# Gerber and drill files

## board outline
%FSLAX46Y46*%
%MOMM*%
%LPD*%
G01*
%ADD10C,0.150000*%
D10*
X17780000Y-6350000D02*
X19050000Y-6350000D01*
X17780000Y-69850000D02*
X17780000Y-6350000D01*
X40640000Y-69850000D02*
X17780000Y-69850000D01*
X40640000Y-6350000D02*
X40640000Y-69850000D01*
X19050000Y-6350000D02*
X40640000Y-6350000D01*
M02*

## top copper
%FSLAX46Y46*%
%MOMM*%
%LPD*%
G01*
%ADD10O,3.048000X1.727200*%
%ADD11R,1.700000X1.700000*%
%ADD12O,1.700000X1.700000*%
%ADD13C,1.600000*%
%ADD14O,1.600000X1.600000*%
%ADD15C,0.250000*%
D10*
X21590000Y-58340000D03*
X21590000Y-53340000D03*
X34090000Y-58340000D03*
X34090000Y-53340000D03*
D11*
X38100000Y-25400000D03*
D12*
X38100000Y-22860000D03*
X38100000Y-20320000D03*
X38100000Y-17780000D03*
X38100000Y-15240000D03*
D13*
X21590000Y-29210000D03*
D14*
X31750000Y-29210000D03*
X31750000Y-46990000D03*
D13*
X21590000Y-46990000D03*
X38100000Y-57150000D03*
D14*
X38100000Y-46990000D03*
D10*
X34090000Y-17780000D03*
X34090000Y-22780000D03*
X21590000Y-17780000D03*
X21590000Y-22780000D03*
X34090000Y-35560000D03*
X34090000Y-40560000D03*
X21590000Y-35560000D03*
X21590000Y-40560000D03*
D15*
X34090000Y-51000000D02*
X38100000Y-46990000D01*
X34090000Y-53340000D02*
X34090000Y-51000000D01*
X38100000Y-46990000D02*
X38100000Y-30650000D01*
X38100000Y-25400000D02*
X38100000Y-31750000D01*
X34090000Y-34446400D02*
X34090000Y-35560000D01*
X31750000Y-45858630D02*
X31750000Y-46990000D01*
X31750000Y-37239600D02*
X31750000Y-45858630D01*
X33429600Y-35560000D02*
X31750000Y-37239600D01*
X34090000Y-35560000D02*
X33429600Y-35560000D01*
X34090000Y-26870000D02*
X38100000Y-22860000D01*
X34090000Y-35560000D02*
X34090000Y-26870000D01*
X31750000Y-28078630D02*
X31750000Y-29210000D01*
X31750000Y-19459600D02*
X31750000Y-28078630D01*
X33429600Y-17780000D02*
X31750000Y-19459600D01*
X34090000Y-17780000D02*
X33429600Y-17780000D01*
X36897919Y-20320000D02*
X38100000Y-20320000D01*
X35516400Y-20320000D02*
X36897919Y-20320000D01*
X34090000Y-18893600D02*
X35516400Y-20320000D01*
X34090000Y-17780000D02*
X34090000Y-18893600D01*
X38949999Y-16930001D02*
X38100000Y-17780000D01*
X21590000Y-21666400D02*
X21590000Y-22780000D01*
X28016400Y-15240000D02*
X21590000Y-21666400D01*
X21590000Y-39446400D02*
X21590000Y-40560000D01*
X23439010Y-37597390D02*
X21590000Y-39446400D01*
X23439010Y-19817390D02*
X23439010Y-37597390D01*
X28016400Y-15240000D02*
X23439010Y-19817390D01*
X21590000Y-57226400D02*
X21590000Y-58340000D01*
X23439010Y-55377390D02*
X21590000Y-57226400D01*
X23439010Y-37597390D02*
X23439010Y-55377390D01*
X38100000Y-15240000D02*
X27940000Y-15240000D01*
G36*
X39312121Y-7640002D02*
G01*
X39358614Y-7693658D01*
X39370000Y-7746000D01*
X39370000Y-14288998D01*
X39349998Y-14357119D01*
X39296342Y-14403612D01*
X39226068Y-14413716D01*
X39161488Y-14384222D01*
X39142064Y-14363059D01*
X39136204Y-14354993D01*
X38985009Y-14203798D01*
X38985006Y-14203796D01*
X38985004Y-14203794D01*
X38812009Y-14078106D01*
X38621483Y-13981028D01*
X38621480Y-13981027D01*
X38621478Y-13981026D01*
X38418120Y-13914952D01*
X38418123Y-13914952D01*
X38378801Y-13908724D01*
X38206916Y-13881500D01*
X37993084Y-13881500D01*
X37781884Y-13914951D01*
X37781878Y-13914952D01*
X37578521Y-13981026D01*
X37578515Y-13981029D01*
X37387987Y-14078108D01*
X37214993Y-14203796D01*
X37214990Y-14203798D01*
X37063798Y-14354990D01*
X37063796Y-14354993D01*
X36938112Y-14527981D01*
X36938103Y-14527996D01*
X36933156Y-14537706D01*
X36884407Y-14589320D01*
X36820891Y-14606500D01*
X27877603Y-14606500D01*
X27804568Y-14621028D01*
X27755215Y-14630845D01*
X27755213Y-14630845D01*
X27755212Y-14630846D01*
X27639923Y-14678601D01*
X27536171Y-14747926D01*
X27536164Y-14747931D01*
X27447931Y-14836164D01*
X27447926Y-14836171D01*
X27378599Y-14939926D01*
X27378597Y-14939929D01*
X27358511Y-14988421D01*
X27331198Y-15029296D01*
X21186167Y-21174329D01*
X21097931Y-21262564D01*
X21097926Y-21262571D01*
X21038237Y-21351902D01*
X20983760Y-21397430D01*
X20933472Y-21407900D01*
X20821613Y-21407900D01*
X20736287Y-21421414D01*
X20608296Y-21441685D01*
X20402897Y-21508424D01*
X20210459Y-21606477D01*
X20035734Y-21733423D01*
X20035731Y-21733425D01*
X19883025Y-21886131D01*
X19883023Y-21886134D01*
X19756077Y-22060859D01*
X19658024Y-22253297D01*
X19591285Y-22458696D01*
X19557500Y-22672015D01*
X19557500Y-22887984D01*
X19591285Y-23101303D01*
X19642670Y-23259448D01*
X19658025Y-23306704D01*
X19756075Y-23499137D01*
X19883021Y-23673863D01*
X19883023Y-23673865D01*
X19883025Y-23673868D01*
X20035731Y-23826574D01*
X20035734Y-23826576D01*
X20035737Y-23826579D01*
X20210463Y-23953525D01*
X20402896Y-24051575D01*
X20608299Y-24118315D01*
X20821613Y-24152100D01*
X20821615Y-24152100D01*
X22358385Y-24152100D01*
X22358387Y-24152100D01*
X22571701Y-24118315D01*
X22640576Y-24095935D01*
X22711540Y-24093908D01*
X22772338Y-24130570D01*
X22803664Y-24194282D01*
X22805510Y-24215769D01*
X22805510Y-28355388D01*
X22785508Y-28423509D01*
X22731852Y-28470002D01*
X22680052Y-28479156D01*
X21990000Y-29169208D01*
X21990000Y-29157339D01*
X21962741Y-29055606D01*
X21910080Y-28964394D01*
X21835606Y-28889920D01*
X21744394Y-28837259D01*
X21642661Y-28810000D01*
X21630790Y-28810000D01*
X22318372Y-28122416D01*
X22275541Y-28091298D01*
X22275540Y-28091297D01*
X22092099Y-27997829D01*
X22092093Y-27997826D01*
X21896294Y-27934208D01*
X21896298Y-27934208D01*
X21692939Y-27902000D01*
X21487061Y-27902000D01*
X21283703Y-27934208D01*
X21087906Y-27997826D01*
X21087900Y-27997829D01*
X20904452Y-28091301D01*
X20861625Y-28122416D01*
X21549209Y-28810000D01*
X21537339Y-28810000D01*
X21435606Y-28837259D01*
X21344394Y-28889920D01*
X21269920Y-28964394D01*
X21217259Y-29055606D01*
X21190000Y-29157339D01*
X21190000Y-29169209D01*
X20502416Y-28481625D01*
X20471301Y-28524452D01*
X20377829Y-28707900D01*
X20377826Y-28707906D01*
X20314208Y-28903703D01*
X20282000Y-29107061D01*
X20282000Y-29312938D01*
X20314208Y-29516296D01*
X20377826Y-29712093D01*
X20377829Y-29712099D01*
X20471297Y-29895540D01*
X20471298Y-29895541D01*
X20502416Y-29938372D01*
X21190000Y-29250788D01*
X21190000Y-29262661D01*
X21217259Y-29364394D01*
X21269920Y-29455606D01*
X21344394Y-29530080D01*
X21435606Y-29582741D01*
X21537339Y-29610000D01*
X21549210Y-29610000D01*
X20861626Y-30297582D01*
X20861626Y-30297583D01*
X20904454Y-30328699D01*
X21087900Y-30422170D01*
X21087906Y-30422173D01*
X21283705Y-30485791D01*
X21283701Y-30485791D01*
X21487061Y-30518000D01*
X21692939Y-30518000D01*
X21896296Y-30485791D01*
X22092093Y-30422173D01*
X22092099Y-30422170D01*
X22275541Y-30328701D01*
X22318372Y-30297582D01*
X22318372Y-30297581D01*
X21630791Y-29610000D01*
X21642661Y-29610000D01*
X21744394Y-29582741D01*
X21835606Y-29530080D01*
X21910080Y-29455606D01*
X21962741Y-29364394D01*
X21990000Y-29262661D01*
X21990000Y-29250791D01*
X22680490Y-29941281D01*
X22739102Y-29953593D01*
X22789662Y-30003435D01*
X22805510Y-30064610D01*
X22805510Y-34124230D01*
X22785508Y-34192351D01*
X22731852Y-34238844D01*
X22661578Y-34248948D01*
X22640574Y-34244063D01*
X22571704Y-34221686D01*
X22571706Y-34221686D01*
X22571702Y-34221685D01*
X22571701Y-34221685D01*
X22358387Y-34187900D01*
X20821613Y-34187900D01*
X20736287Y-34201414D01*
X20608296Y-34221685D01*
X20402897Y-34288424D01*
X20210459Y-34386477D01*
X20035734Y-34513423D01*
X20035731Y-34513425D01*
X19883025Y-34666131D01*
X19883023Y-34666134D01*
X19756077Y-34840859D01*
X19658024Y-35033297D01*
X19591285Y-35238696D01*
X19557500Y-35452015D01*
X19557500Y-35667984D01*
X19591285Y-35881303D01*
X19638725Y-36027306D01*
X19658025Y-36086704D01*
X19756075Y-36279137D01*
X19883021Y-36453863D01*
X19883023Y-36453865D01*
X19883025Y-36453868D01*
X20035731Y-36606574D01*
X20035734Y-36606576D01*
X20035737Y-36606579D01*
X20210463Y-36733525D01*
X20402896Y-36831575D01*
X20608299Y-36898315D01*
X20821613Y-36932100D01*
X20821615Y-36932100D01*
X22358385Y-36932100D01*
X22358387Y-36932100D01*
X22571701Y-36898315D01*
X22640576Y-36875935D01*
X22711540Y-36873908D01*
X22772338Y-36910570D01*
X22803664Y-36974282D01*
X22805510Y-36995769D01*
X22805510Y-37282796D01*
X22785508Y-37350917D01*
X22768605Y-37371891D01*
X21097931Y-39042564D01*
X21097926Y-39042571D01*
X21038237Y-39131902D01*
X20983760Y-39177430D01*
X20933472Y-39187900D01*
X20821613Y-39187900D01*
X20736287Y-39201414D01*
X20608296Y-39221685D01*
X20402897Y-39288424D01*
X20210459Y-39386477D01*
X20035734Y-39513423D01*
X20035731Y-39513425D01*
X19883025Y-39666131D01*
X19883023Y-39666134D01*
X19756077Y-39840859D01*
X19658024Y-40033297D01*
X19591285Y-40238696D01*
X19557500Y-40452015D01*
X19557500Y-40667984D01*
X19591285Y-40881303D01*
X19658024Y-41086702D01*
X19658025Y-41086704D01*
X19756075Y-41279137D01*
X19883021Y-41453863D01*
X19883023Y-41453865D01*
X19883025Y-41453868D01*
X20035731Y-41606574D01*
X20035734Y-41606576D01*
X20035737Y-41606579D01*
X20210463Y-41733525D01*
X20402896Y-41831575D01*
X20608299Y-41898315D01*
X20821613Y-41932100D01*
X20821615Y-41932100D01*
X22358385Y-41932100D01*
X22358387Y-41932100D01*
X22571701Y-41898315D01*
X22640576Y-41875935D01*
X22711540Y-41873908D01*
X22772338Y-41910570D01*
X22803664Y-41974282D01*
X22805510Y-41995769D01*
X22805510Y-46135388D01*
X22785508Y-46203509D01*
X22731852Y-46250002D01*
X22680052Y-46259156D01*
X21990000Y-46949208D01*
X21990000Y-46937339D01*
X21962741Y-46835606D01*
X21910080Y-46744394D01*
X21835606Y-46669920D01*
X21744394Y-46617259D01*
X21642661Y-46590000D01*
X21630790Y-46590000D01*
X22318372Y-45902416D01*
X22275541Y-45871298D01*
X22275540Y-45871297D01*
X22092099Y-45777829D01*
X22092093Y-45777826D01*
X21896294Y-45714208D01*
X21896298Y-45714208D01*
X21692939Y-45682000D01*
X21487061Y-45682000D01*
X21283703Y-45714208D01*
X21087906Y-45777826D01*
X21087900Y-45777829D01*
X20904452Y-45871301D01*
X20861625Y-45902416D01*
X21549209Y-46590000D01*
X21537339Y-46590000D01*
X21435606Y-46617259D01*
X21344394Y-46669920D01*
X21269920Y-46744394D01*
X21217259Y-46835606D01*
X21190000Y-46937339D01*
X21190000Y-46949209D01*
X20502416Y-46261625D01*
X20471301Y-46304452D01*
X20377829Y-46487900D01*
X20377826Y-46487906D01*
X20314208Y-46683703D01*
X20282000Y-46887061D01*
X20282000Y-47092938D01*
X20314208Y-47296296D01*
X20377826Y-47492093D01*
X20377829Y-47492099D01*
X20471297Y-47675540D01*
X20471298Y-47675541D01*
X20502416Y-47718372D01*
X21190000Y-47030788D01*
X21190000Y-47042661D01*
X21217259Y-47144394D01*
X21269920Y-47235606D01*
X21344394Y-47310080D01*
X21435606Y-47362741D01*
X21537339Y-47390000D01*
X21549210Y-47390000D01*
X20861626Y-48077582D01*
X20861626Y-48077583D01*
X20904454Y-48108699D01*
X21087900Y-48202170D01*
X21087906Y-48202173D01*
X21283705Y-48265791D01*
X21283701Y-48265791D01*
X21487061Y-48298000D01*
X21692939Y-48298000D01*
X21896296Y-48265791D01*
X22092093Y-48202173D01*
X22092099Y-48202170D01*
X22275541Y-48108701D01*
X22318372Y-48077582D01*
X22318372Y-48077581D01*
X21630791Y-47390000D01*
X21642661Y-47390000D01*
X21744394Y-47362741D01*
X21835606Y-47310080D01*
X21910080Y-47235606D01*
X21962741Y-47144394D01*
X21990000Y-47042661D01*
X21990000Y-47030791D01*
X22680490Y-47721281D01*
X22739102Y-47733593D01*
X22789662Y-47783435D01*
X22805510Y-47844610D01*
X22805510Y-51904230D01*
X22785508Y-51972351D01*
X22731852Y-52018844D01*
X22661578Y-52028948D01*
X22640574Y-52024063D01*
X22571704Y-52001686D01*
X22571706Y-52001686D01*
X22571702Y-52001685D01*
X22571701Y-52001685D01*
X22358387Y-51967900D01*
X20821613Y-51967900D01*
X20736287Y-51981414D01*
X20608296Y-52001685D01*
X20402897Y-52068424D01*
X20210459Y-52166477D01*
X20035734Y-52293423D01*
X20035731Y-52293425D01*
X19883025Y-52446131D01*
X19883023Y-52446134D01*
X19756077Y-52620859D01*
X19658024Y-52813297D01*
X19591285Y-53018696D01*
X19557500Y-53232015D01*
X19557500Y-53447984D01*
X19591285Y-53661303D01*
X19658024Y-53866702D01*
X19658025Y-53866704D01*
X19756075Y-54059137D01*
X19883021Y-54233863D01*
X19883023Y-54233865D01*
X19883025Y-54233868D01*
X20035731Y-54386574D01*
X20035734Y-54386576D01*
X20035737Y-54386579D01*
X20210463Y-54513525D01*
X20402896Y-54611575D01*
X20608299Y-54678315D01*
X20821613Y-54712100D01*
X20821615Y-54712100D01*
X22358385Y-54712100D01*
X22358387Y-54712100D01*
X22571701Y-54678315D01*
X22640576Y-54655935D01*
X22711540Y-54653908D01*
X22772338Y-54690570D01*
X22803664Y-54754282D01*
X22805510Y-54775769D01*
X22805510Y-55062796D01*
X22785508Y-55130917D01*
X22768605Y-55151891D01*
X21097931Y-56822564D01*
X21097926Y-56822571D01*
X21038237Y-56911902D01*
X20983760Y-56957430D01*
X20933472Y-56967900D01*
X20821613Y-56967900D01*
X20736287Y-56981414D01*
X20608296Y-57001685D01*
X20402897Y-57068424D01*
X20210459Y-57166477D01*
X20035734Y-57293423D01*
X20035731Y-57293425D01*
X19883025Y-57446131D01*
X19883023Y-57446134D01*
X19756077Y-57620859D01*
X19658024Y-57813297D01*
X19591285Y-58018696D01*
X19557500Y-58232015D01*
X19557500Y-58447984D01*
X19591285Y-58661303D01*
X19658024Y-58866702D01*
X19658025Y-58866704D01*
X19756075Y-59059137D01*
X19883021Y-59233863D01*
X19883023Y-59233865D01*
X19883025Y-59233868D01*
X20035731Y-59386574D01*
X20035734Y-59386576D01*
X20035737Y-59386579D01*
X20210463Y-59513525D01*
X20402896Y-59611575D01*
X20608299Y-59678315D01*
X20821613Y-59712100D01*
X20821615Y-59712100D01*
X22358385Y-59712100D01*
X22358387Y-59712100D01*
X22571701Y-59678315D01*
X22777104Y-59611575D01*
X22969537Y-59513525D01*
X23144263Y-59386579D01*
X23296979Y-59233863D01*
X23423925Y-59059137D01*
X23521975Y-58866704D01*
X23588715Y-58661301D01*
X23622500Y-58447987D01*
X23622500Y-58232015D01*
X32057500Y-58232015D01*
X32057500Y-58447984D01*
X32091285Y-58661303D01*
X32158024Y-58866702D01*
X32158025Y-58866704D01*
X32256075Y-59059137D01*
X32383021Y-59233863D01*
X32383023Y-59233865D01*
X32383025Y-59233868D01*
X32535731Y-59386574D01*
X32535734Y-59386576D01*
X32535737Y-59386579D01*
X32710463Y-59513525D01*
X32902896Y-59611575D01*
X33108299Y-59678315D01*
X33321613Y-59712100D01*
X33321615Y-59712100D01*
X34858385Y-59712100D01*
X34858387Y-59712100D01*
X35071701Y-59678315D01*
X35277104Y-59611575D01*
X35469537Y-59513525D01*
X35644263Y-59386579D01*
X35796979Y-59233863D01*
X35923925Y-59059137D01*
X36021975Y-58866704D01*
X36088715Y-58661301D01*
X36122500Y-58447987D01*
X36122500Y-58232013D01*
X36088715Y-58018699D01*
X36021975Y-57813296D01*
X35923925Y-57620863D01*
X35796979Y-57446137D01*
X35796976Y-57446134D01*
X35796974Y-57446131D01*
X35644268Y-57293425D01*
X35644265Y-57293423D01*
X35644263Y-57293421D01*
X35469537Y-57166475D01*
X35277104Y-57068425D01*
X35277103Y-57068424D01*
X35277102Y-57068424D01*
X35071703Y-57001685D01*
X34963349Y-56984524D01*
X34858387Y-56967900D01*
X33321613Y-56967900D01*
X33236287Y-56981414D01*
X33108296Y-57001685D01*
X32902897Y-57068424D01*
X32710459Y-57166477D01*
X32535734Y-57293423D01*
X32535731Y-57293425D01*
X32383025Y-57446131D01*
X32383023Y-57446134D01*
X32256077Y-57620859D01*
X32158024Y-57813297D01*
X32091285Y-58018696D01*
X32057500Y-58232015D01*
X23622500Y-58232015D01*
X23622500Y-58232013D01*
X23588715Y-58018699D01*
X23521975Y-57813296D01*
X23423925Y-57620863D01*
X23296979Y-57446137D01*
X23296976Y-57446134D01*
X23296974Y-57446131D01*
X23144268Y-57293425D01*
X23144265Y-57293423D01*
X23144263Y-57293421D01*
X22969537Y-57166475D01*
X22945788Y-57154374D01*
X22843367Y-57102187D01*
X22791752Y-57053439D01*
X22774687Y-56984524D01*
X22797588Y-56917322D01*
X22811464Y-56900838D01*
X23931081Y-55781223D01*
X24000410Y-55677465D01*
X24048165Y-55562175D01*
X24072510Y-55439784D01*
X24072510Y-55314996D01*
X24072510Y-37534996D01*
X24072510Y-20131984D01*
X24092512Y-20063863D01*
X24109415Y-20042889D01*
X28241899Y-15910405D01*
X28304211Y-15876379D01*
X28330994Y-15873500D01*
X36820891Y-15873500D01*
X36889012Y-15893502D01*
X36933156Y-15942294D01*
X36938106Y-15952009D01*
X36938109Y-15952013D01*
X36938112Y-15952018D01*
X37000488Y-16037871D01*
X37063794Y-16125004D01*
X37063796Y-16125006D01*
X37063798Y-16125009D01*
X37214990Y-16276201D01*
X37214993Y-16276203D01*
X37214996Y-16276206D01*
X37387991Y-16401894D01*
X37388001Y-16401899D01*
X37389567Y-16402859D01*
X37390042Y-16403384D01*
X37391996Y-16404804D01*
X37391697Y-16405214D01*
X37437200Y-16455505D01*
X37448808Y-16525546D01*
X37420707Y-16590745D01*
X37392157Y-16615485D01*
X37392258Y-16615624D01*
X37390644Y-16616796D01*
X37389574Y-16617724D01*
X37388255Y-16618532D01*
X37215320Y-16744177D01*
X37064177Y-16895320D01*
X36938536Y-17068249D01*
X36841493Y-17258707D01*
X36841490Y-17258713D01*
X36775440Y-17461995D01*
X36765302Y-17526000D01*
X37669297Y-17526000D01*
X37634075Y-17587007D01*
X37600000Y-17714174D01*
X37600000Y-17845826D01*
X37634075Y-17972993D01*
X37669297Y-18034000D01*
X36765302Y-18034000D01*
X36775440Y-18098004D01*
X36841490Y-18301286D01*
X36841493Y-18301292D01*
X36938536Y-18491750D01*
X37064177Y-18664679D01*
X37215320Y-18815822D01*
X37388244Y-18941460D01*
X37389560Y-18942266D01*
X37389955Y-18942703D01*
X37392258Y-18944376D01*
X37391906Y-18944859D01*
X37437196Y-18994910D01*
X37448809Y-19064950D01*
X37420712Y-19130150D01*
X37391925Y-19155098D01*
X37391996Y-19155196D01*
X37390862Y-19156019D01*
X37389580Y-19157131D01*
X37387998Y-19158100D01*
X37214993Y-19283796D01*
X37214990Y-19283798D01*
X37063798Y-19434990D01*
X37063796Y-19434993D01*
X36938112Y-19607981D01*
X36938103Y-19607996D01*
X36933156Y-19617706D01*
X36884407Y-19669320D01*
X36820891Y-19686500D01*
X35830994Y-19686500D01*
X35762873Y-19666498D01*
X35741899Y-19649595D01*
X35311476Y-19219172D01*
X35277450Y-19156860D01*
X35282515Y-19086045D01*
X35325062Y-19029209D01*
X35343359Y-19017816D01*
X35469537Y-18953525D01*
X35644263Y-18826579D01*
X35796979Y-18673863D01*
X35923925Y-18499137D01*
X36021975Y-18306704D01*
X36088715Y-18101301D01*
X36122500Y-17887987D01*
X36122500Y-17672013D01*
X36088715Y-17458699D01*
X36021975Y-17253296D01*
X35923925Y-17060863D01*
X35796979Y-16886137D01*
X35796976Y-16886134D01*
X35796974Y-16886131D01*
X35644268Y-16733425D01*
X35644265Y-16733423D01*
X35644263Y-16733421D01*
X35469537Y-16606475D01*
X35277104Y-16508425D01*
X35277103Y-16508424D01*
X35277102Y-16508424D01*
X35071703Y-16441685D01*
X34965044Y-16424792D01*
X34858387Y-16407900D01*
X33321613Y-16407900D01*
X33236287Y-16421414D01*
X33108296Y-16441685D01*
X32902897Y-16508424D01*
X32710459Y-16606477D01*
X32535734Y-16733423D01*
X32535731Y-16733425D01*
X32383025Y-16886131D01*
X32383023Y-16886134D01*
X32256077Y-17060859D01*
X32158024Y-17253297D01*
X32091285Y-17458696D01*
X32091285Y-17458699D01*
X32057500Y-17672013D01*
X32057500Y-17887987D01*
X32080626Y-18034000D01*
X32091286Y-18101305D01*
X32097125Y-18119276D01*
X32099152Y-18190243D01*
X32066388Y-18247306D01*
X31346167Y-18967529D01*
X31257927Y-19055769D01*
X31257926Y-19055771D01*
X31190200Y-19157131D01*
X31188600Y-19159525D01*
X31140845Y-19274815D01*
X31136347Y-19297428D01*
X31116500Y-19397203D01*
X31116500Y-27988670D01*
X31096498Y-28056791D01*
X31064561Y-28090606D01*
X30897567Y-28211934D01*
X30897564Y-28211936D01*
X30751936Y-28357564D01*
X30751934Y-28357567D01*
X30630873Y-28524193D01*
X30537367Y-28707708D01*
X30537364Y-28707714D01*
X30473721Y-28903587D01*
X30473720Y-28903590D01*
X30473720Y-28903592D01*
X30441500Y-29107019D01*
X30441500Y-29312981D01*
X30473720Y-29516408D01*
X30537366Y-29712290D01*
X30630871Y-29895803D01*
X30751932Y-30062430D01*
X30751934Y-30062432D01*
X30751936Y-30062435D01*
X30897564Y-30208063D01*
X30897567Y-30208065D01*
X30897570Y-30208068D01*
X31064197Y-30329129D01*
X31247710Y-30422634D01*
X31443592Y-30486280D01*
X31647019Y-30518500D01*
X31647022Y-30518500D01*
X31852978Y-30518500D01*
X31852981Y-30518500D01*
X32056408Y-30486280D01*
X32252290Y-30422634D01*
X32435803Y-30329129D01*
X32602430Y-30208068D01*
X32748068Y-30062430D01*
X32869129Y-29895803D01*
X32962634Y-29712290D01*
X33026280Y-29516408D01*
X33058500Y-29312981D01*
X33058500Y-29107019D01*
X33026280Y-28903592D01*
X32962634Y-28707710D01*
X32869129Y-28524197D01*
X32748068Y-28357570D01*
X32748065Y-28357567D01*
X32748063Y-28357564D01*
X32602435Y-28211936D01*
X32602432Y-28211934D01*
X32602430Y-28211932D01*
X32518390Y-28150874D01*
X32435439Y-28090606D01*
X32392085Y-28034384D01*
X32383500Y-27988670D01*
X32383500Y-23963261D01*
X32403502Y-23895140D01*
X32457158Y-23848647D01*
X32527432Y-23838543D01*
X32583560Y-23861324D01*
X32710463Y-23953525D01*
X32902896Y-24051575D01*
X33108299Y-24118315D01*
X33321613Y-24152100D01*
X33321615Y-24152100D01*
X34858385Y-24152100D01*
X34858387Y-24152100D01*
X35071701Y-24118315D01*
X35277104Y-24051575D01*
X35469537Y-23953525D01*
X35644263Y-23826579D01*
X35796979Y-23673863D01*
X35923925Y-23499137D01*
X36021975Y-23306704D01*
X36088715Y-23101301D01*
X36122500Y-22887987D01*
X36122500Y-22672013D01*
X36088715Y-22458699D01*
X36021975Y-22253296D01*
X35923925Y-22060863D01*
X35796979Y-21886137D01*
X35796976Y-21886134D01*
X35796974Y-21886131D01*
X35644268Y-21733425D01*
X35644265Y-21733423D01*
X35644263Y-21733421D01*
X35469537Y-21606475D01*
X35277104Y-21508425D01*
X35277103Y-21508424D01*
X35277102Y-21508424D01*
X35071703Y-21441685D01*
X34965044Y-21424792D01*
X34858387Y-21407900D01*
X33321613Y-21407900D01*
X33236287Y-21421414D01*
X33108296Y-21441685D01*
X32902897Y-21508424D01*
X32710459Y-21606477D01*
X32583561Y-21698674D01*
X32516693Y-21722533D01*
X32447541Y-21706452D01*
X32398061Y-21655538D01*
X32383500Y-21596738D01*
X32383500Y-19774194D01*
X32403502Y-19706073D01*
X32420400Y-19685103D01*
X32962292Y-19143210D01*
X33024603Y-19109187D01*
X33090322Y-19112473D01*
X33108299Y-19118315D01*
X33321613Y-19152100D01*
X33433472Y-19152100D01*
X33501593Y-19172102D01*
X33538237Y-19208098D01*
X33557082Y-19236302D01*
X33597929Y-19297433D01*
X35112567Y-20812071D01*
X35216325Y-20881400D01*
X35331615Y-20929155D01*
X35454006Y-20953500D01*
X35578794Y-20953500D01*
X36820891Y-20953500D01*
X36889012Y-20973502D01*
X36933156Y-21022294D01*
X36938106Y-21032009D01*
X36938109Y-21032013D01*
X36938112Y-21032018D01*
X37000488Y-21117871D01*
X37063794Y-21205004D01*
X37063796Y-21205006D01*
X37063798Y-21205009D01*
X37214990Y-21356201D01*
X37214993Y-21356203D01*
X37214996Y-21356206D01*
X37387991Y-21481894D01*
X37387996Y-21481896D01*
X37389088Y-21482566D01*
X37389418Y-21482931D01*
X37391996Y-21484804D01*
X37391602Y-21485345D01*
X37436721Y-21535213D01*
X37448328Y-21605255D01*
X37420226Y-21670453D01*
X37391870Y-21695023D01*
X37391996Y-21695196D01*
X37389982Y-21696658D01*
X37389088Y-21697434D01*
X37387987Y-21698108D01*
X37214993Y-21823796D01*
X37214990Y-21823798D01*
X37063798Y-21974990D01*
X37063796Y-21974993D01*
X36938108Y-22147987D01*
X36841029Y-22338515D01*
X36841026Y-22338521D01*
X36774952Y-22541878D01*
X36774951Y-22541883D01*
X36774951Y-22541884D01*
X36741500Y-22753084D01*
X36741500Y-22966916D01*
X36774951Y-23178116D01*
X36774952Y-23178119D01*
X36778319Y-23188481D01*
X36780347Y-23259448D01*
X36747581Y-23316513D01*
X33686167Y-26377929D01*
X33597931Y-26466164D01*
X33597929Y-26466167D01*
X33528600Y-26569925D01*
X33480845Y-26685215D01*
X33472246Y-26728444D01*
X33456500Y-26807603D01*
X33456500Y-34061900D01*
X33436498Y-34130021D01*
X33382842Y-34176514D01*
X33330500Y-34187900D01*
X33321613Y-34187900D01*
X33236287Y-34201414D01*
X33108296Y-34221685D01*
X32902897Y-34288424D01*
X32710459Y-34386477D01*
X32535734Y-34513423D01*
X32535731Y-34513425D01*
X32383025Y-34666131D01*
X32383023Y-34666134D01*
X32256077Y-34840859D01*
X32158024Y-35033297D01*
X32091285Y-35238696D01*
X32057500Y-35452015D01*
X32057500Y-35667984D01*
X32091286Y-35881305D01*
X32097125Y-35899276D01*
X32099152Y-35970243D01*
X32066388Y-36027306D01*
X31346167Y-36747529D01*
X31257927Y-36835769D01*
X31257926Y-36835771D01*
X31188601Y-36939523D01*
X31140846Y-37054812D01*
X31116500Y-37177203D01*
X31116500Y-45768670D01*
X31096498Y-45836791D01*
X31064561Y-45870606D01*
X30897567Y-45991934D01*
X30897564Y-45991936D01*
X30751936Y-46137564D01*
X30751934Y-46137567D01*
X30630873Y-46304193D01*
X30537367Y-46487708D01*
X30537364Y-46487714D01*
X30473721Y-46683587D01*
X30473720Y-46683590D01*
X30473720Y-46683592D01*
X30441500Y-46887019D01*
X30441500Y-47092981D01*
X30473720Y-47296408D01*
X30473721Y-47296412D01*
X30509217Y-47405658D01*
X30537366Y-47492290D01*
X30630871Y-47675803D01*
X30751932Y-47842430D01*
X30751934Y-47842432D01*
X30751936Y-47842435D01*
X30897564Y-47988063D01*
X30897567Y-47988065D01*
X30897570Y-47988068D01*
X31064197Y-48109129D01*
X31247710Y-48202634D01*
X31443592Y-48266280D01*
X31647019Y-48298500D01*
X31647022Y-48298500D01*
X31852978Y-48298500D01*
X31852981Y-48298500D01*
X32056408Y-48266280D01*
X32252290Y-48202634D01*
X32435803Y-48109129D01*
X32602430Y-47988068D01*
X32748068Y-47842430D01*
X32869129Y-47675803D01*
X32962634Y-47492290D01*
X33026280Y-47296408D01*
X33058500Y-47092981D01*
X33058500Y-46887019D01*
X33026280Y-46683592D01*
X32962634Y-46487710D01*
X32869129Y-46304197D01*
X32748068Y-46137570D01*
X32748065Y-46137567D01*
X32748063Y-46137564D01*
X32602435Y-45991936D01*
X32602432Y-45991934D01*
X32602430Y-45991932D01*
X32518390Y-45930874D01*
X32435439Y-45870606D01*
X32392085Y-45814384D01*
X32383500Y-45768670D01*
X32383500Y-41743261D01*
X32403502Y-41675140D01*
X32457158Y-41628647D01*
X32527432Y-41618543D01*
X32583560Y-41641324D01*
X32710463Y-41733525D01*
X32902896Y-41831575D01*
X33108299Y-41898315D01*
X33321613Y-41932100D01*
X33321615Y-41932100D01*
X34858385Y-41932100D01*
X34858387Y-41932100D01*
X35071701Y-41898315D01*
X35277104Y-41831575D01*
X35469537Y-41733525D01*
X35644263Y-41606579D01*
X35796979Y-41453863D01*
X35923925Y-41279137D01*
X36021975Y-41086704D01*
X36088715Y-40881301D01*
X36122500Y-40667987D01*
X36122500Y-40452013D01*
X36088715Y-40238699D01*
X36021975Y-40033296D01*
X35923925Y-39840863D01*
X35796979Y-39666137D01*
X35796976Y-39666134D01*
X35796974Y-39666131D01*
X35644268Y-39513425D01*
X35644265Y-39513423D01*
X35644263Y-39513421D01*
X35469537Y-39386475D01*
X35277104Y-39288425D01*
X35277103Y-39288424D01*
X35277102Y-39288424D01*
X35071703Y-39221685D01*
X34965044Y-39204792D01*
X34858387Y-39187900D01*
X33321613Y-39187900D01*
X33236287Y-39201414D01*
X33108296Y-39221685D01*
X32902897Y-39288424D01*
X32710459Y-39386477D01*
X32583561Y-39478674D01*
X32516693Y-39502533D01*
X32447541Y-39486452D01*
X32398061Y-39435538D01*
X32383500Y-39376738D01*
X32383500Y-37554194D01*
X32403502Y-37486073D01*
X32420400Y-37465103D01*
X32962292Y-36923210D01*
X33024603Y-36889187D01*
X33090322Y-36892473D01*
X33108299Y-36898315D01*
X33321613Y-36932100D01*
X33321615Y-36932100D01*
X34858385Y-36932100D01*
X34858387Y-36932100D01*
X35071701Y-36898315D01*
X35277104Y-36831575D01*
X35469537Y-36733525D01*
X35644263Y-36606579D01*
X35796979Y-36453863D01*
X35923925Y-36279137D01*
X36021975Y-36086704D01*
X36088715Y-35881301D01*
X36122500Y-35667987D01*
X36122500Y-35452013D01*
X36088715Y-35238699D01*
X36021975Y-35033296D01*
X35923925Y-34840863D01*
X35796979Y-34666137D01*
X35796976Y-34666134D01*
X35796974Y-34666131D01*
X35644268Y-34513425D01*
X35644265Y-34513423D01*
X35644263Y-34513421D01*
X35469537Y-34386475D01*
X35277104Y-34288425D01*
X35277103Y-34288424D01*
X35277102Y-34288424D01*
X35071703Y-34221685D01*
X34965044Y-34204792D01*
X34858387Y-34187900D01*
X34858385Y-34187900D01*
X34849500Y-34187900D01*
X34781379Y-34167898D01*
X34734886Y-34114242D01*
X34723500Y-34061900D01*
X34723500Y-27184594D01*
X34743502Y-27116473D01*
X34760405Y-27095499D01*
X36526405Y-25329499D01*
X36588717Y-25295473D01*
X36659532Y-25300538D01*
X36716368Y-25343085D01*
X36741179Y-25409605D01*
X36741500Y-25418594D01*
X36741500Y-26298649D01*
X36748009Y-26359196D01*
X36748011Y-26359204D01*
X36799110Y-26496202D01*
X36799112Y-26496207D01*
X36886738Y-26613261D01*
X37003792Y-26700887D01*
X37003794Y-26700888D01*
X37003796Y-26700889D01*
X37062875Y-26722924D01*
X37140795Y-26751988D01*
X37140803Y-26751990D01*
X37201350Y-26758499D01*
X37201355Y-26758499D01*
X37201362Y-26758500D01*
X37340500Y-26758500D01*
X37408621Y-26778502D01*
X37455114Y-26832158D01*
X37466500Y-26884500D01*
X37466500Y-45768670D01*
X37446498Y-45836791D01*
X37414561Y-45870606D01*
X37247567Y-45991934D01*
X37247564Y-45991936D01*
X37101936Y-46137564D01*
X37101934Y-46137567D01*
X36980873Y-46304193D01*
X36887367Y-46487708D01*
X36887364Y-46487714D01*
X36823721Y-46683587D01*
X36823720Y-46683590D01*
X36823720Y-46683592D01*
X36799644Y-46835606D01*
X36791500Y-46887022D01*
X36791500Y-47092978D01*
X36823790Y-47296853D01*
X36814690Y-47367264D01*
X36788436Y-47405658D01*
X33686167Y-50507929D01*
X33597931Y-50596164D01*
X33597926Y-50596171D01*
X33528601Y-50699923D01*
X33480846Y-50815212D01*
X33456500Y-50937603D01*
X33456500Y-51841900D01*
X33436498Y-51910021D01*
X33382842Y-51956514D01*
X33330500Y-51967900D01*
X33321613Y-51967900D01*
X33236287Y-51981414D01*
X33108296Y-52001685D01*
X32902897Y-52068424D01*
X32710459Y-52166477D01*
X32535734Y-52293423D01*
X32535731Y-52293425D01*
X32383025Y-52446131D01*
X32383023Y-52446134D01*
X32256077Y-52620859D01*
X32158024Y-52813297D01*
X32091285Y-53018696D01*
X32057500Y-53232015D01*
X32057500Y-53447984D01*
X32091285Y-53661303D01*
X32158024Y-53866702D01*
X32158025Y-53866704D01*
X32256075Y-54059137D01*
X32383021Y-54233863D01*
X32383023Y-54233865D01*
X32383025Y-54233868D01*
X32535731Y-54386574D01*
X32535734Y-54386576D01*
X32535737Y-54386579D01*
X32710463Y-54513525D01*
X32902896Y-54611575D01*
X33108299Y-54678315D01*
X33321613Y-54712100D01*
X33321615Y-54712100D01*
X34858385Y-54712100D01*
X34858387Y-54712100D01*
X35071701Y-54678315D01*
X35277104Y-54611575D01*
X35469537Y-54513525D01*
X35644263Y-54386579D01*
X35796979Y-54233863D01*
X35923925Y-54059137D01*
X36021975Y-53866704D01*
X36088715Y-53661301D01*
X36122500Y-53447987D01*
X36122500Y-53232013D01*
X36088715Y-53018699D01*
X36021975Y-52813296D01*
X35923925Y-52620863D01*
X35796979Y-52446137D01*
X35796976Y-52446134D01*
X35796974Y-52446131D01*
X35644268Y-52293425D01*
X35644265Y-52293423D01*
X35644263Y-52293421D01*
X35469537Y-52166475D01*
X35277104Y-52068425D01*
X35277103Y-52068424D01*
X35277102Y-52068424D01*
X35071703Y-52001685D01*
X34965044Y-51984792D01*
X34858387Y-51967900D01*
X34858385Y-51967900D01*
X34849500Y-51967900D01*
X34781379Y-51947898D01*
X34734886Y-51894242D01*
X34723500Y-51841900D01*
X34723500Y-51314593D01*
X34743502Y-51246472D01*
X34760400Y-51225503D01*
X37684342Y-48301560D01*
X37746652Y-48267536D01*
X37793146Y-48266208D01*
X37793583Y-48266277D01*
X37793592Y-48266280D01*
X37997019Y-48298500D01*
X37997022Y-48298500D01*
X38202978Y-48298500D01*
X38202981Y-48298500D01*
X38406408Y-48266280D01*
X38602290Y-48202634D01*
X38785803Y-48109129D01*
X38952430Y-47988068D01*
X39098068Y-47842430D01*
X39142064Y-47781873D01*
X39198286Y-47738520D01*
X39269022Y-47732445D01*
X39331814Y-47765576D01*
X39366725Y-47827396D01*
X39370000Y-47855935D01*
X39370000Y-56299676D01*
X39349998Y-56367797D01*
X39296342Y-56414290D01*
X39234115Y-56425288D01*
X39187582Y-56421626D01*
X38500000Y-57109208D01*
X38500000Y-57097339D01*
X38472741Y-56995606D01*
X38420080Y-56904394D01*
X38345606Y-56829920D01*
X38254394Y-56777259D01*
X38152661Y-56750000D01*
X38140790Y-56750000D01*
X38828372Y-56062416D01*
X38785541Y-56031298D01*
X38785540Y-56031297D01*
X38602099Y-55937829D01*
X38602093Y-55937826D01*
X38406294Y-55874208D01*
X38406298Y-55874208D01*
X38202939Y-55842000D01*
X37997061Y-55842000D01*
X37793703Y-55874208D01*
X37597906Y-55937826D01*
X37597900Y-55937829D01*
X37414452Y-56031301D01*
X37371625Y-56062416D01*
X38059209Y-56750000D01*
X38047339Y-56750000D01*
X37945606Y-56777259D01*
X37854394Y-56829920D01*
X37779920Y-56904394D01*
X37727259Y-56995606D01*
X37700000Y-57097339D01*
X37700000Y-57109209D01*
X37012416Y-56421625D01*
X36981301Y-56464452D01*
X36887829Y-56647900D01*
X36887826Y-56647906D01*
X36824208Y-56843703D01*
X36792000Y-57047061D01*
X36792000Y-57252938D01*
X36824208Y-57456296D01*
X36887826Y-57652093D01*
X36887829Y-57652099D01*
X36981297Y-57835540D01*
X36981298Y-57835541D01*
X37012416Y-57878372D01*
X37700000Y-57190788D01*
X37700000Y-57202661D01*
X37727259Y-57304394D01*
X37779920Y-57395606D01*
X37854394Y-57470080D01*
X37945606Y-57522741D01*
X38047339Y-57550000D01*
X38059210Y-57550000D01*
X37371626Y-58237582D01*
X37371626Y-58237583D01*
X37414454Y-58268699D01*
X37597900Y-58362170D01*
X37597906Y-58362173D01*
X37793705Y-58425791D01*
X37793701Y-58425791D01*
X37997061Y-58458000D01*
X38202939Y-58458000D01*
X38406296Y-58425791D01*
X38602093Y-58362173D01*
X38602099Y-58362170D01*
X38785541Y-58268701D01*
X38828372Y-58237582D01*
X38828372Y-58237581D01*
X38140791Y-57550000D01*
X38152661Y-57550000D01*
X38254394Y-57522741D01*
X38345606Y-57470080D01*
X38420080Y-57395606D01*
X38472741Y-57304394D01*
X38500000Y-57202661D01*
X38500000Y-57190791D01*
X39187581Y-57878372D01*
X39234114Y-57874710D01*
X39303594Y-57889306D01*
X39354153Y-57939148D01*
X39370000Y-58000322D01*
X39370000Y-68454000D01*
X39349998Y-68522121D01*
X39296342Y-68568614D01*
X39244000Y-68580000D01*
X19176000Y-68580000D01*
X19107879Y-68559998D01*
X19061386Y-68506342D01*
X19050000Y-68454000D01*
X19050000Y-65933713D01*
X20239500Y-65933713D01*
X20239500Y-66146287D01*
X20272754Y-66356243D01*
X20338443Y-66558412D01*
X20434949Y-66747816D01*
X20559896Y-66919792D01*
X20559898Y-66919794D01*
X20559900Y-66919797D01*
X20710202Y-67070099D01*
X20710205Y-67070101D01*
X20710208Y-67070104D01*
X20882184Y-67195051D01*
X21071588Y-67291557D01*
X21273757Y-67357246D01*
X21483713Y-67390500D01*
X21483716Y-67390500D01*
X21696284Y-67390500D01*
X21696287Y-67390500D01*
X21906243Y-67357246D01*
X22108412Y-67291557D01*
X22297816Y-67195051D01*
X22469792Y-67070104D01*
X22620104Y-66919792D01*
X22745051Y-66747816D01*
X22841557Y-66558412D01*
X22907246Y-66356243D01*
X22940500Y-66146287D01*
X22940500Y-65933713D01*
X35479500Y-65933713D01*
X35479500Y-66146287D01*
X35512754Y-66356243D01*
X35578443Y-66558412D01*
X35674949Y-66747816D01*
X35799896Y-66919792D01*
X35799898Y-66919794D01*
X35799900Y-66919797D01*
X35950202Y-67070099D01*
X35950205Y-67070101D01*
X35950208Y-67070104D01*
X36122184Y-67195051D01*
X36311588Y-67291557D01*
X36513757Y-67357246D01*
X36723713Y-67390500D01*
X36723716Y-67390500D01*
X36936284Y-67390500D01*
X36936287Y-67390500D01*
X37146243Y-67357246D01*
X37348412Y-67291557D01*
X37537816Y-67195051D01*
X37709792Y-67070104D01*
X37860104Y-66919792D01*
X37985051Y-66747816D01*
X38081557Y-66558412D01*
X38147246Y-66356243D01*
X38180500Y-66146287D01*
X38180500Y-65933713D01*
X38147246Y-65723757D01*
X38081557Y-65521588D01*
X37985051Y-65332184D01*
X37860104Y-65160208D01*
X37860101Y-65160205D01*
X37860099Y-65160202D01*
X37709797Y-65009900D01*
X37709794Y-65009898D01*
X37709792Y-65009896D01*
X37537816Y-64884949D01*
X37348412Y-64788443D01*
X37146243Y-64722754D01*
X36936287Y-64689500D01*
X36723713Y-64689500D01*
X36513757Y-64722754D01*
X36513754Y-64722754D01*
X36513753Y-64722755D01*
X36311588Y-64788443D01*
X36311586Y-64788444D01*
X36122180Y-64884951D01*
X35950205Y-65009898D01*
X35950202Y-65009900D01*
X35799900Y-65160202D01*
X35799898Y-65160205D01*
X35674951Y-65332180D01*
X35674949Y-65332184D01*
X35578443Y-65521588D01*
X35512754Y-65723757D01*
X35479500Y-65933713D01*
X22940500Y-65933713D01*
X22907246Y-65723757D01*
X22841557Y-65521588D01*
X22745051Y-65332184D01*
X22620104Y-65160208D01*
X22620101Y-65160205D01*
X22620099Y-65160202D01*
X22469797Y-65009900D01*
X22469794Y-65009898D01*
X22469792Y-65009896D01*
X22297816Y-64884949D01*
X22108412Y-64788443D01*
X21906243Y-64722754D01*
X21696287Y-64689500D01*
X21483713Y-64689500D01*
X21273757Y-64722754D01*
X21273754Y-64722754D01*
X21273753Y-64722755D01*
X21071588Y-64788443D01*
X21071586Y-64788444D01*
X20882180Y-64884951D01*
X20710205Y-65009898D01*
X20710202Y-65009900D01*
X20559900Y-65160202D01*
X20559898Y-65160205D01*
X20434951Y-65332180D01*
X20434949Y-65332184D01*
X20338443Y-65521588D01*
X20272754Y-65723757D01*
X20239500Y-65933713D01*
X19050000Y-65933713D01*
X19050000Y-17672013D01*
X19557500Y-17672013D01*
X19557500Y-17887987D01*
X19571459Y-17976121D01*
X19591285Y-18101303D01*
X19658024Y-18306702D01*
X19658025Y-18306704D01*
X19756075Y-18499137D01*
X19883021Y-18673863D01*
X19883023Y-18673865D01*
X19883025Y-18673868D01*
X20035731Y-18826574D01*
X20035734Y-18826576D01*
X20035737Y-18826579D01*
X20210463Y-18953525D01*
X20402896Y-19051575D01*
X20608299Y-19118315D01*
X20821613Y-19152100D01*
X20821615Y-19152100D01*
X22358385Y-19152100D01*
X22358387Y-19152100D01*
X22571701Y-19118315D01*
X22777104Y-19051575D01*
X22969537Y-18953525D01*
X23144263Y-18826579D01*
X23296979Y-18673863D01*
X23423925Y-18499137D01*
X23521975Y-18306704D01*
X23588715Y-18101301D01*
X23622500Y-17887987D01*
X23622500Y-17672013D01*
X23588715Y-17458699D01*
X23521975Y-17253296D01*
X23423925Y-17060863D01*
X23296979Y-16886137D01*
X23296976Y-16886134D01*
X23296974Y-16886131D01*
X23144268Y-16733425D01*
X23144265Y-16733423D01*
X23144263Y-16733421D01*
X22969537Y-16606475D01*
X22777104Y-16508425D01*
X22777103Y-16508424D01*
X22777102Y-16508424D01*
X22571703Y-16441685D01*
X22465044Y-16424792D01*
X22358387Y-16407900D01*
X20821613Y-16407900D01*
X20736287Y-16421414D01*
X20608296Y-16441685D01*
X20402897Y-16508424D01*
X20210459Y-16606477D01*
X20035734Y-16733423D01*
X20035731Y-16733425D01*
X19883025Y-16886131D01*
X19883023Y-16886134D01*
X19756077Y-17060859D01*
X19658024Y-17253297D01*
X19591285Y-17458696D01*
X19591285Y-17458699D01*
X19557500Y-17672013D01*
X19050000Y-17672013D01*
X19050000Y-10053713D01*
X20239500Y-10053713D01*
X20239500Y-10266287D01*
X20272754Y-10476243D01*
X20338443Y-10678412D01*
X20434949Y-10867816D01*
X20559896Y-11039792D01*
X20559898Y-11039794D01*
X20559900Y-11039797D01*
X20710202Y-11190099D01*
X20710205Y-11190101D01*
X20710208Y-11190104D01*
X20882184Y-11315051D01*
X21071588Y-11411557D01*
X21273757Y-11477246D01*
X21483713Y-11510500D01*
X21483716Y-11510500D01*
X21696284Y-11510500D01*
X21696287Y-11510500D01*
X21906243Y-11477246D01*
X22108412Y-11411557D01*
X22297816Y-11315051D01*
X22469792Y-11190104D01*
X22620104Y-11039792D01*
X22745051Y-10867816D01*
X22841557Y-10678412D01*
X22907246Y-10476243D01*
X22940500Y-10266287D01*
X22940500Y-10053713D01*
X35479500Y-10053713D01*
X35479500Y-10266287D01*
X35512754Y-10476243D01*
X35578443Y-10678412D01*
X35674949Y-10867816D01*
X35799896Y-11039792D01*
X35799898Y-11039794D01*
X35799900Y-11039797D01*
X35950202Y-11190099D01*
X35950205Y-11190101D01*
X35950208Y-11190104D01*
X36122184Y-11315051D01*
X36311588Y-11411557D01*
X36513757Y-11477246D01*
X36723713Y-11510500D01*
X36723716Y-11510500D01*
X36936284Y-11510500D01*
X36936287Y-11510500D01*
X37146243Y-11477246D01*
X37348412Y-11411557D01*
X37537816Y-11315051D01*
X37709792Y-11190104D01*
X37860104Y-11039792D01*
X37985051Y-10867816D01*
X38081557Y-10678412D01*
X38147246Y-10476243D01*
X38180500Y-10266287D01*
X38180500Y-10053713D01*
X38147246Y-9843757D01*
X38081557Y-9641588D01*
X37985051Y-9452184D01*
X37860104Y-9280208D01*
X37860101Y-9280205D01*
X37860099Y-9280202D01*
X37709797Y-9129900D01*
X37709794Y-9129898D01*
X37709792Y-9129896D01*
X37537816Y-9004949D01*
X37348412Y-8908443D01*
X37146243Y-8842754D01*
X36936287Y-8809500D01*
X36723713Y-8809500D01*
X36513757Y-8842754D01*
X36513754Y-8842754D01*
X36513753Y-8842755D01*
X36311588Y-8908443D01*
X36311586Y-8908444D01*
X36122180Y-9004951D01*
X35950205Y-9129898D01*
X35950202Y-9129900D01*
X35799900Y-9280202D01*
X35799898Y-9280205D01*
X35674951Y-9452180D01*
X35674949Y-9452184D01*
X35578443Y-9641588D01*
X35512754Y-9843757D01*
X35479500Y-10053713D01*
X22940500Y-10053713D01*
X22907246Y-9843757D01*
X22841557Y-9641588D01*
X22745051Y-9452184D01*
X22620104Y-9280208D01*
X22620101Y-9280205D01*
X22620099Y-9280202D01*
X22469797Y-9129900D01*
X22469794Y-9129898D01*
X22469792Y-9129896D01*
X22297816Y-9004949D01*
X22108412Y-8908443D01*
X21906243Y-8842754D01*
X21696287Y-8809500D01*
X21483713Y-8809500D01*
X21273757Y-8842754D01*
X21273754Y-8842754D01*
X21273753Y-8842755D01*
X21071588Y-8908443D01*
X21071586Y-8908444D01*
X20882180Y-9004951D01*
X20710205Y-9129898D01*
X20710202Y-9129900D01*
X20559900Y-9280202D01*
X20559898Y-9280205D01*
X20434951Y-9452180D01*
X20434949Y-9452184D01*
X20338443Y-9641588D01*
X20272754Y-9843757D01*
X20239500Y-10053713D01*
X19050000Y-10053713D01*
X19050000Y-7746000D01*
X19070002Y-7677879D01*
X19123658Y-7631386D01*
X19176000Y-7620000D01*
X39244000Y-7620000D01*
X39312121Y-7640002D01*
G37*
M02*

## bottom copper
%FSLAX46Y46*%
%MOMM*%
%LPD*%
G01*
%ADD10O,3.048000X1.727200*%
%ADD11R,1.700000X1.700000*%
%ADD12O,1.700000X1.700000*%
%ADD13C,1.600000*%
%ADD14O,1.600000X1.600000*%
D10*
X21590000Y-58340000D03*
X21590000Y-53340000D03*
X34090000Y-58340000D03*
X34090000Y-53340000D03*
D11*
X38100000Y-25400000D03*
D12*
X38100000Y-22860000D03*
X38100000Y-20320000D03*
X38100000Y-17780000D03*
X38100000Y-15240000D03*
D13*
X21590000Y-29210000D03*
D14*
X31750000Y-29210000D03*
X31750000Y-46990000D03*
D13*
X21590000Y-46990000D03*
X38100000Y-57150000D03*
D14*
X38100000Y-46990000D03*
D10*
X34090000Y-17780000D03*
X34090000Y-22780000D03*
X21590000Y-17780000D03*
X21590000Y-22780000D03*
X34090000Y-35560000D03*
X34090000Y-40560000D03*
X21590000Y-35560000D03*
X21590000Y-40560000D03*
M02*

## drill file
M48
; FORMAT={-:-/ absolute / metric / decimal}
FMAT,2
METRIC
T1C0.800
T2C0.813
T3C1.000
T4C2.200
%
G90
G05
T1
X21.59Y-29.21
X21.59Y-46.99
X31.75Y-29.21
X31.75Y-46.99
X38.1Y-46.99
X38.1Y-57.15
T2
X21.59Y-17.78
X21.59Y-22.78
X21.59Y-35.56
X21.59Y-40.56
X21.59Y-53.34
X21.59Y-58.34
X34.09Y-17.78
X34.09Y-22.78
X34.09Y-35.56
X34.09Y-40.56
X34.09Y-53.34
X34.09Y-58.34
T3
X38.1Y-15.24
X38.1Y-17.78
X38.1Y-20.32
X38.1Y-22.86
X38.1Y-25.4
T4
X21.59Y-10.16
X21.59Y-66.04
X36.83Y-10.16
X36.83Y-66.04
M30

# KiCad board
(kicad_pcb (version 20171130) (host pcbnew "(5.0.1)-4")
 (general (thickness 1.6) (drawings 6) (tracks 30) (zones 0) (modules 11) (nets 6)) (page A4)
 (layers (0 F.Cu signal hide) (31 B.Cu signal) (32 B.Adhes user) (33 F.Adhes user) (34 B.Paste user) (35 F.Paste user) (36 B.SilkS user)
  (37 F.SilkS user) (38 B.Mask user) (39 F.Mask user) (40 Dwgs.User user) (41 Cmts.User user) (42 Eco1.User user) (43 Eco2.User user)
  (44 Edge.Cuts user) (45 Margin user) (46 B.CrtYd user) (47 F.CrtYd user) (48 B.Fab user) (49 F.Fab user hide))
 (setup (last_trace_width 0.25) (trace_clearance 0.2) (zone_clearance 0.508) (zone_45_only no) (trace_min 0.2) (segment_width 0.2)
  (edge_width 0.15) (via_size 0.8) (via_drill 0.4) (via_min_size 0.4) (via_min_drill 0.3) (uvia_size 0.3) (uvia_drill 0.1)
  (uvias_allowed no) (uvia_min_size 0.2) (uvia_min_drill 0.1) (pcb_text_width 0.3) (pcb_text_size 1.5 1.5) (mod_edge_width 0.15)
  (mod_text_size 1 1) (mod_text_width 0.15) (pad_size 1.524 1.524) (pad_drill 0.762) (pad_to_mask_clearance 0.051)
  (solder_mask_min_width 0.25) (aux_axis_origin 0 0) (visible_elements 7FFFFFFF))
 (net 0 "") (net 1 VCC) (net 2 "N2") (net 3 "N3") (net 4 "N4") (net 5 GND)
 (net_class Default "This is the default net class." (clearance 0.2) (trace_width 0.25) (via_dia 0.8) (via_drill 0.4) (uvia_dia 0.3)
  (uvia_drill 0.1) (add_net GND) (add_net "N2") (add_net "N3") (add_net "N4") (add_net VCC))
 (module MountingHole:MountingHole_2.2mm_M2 (layer F.Cu) (at 36.83 66.04)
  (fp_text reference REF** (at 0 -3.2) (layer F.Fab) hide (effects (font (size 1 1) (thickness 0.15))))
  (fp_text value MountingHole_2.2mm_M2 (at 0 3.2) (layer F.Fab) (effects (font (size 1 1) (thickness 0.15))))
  (pad 1 np_thru_hole circle (at 0 0) (size 2.2 2.2) (drill 2.2) (layers *.Cu *.Mask)))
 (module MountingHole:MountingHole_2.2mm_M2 (layer F.Cu) (at 21.59 66.04)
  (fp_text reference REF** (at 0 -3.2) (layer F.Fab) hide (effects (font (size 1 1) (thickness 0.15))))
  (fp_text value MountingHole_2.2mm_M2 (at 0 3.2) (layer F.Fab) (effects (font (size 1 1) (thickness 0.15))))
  (pad 1 np_thru_hole circle (at 0 0) (size 2.2 2.2) (drill 2.2) (layers *.Cu *.Mask)))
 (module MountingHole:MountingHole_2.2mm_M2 (layer F.Cu) (at 36.83 10.16)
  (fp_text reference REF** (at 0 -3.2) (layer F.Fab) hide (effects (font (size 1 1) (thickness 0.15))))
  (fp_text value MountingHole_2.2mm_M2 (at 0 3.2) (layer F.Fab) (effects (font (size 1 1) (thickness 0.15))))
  (pad 1 np_thru_hole circle (at 0 0) (size 2.2 2.2) (drill 2.2) (layers *.Cu *.Mask)))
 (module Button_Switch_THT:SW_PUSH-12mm (layer F.Cu) (at 21.59 53.34)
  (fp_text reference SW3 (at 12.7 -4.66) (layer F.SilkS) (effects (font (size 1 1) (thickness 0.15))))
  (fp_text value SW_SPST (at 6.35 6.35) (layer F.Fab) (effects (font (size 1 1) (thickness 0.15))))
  (pad 2 thru_hole oval (at 0 5) (size 3.048 1.7272) (drill 0.8128) (layers *.Cu *.Mask) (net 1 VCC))
  (pad 1 thru_hole oval (at 0 0) (size 3.048 1.7272) (drill 0.8128) (layers *.Cu *.Mask) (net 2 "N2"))
  (pad 2 thru_hole oval (at 12.5 5) (size 3.048 1.7272) (drill 0.8128) (layers *.Cu *.Mask) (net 1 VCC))
  (pad 1 thru_hole oval (at 12.5 0) (size 3.048 1.7272) (drill 0.8128) (layers *.Cu *.Mask) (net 2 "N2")))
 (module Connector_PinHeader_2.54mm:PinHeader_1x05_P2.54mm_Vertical (layer F.Cu) (at 38.1 25.4 180)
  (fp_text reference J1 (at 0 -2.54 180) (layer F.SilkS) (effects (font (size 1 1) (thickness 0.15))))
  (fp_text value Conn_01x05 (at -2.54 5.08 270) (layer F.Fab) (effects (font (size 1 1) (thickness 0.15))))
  (pad 1 thru_hole rect (at 0 0 180) (size 1.7 1.7) (drill 1) (layers *.Cu *.Mask) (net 2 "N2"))
  (pad 2 thru_hole oval (at 0 2.54 180) (size 1.7 1.7) (drill 1) (layers *.Cu *.Mask) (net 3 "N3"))
  (pad 3 thru_hole oval (at 0 5.08 180) (size 1.7 1.7) (drill 1) (layers *.Cu *.Mask) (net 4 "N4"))
  (pad 4 thru_hole oval (at 0 7.62 180) (size 1.7 1.7) (drill 1) (layers *.Cu *.Mask) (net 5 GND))
  (pad 5 thru_hole oval (at 0 10.16 180) (size 1.7 1.7) (drill 1) (layers *.Cu *.Mask) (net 1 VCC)))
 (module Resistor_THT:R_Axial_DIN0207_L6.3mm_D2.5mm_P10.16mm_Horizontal (layer F.Cu) (at 21.59 29.21)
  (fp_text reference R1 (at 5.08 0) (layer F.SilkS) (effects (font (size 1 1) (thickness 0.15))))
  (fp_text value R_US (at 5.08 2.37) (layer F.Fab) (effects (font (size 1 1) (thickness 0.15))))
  (pad 1 thru_hole circle (at 0 0) (size 1.6 1.6) (drill 0.8) (layers *.Cu *.Mask) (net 5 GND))
  (pad 2 thru_hole oval (at 10.16 0) (size 1.6 1.6) (drill 0.8) (layers *.Cu *.Mask) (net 4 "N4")))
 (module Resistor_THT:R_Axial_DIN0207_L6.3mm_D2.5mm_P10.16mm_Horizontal (layer F.Cu) (at 21.59 46.99)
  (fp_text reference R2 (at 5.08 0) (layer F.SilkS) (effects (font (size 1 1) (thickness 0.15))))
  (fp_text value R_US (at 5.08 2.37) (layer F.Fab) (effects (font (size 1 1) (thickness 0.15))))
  (pad 2 thru_hole oval (at 10.16 0) (size 1.6 1.6) (drill 0.8) (layers *.Cu *.Mask) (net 3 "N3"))
  (pad 1 thru_hole circle (at 0 0) (size 1.6 1.6) (drill 0.8) (layers *.Cu *.Mask) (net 5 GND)))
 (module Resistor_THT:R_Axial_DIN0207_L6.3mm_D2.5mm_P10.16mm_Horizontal (layer F.Cu) (at 38.1 57.15 90)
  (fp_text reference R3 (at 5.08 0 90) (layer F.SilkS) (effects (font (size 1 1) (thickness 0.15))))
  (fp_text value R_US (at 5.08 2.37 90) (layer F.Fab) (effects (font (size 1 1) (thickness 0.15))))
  (pad 1 thru_hole circle (at 0 0 90) (size 1.6 1.6) (drill 0.8) (layers *.Cu *.Mask) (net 5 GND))
  (pad 2 thru_hole oval (at 10.16 0 90) (size 1.6 1.6) (drill 0.8) (layers *.Cu *.Mask) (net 2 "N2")))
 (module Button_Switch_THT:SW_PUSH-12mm (layer F.Cu) (at 21.59 17.78)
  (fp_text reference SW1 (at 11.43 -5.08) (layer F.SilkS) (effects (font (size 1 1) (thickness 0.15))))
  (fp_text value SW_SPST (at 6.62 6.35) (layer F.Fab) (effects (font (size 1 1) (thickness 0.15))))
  (pad 1 thru_hole oval (at 12.5 0) (size 3.048 1.7272) (drill 0.8128) (layers *.Cu *.Mask) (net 4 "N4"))
  (pad 2 thru_hole oval (at 12.5 5) (size 3.048 1.7272) (drill 0.8128) (layers *.Cu *.Mask) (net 1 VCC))
  (pad 1 thru_hole oval (at 0 0) (size 3.048 1.7272) (drill 0.8128) (layers *.Cu *.Mask) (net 4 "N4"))
  (pad 2 thru_hole oval (at 0 5) (size 3.048 1.7272) (drill 0.8128) (layers *.Cu *.Mask) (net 1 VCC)))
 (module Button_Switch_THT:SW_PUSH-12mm (layer F.Cu) (at 21.59 35.56)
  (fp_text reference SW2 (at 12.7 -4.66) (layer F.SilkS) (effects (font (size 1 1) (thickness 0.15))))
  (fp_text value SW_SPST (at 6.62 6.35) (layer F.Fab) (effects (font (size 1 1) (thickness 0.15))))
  (pad 1 thru_hole oval (at 12.5 0) (size 3.048 1.7272) (drill 0.8128) (layers *.Cu *.Mask) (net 3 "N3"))
  (pad 2 thru_hole oval (at 12.5 5) (size 3.048 1.7272) (drill 0.8128) (layers *.Cu *.Mask) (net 1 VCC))
  (pad 1 thru_hole oval (at 0 0) (size 3.048 1.7272) (drill 0.8128) (layers *.Cu *.Mask) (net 3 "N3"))
  (pad 2 thru_hole oval (at 0 5) (size 3.048 1.7272) (drill 0.8128) (layers *.Cu *.Mask) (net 1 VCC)))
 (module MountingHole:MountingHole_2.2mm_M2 (layer F.Cu) (at 21.59 10.16)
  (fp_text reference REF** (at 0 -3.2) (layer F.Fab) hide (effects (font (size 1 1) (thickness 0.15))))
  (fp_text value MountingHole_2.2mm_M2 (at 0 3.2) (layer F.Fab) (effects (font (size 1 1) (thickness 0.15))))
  (pad 1 np_thru_hole circle (at 0 0) (size 2.2 2.2) (drill 2.2) (layers *.Cu *.Mask)))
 (gr_line (start 17.78 6.35) (end 19.05 6.35) (layer Edge.Cuts) (width 0.15))
 (gr_line (start 17.78 69.85) (end 17.78 6.35) (layer Edge.Cuts) (width 0.15))
 (gr_line (start 40.64 69.85) (end 17.78 69.85) (layer Edge.Cuts) (width 0.15))
 (gr_line (start 40.64 6.35) (end 40.64 69.85) (layer Edge.Cuts) (width 0.15))
 (gr_line (start 19.05 6.35) (end 40.64 6.35) (layer Edge.Cuts) (width 0.15))
 (segment (start 34.09 51) (end 38.1 46.99) (width 0.25) (layer F.Cu) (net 2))
 (segment (start 34.09 53.34) (end 34.09 51) (width 0.25) (layer F.Cu) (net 2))
 (segment (start 38.1 46.99) (end 38.1 30.65) (width 0.25) (layer F.Cu) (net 2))
 (segment (start 38.1 25.4) (end 38.1 31.75) (width 0.25) (layer F.Cu) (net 2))
 (segment (start 34.09 34.4464) (end 34.09 35.56) (width 0.25) (layer F.Cu) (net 3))
 (segment (start 31.75 45.85863) (end 31.75 46.99) (width 0.25) (layer F.Cu) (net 3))
 (segment (start 31.75 37.2396) (end 31.75 45.85863) (width 0.25) (layer F.Cu) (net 3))
 (segment (start 33.4296 35.56) (end 31.75 37.2396) (width 0.25) (layer F.Cu) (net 3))
 (segment (start 34.09 35.56) (end 33.4296 35.56) (width 0.25) (layer F.Cu) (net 3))
 (segment (start 34.09 26.87) (end 38.1 22.86) (width 0.25) (layer F.Cu) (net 3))
 (segment (start 34.09 35.56) (end 34.09 26.87) (width 0.25) (layer F.Cu) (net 3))
 (segment (start 31.75 28.07863) (end 31.75 29.21) (width 0.25) (layer F.Cu) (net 4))
 (segment (start 31.75 19.4596) (end 31.75 28.07863) (width 0.25) (layer F.Cu) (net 4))
 (segment (start 33.4296 17.78) (end 31.75 19.4596) (width 0.25) (layer F.Cu) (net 4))
 (segment (start 34.09 17.78) (end 33.4296 17.78) (width 0.25) (layer F.Cu) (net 4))
 (segment (start 36.897919 20.32) (end 38.1 20.32) (width 0.25) (layer F.Cu) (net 4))
 (segment (start 35.5164 20.32) (end 36.897919 20.32) (width 0.25) (layer F.Cu) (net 4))
 (segment (start 34.09 18.8936) (end 35.5164 20.32) (width 0.25) (layer F.Cu) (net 4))
 (segment (start 34.09 17.78) (end 34.09 18.8936) (width 0.25) (layer F.Cu) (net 4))
 (segment (start 38.949999 16.930001) (end 38.1 17.78) (width 0.25) (layer F.Cu) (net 5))
 (segment (start 21.59 21.6664) (end 21.59 22.78) (width 0.25) (layer F.Cu) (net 1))
 (segment (start 28.0164 15.24) (end 21.59 21.6664) (width 0.25) (layer F.Cu) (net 1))
 (segment (start 21.59 39.4464) (end 21.59 40.56) (width 0.25) (layer F.Cu) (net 1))
 (segment (start 23.43901 37.59739) (end 21.59 39.4464) (width 0.25) (layer F.Cu) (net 1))
 (segment (start 23.43901 19.81739) (end 23.43901 37.59739) (width 0.25) (layer F.Cu) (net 1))
 (segment (start 28.0164 15.24) (end 23.43901 19.81739) (width 0.25) (layer F.Cu) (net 1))
 (segment (start 21.59 57.2264) (end 21.59 58.34) (width 0.25) (layer F.Cu) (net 1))
 (segment (start 23.43901 55.37739) (end 21.59 57.2264) (width 0.25) (layer F.Cu) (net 1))
 (segment (start 23.43901 37.59739) (end 23.43901 55.37739) (width 0.25) (layer F.Cu) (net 1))
 (segment (start 38.1 15.24) (end 27.94 15.24) (width 0.25) (layer F.Cu) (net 1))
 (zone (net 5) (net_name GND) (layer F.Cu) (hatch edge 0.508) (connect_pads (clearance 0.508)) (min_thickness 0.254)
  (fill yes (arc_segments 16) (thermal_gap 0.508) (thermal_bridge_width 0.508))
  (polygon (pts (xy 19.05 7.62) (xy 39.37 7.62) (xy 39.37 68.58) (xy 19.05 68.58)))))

